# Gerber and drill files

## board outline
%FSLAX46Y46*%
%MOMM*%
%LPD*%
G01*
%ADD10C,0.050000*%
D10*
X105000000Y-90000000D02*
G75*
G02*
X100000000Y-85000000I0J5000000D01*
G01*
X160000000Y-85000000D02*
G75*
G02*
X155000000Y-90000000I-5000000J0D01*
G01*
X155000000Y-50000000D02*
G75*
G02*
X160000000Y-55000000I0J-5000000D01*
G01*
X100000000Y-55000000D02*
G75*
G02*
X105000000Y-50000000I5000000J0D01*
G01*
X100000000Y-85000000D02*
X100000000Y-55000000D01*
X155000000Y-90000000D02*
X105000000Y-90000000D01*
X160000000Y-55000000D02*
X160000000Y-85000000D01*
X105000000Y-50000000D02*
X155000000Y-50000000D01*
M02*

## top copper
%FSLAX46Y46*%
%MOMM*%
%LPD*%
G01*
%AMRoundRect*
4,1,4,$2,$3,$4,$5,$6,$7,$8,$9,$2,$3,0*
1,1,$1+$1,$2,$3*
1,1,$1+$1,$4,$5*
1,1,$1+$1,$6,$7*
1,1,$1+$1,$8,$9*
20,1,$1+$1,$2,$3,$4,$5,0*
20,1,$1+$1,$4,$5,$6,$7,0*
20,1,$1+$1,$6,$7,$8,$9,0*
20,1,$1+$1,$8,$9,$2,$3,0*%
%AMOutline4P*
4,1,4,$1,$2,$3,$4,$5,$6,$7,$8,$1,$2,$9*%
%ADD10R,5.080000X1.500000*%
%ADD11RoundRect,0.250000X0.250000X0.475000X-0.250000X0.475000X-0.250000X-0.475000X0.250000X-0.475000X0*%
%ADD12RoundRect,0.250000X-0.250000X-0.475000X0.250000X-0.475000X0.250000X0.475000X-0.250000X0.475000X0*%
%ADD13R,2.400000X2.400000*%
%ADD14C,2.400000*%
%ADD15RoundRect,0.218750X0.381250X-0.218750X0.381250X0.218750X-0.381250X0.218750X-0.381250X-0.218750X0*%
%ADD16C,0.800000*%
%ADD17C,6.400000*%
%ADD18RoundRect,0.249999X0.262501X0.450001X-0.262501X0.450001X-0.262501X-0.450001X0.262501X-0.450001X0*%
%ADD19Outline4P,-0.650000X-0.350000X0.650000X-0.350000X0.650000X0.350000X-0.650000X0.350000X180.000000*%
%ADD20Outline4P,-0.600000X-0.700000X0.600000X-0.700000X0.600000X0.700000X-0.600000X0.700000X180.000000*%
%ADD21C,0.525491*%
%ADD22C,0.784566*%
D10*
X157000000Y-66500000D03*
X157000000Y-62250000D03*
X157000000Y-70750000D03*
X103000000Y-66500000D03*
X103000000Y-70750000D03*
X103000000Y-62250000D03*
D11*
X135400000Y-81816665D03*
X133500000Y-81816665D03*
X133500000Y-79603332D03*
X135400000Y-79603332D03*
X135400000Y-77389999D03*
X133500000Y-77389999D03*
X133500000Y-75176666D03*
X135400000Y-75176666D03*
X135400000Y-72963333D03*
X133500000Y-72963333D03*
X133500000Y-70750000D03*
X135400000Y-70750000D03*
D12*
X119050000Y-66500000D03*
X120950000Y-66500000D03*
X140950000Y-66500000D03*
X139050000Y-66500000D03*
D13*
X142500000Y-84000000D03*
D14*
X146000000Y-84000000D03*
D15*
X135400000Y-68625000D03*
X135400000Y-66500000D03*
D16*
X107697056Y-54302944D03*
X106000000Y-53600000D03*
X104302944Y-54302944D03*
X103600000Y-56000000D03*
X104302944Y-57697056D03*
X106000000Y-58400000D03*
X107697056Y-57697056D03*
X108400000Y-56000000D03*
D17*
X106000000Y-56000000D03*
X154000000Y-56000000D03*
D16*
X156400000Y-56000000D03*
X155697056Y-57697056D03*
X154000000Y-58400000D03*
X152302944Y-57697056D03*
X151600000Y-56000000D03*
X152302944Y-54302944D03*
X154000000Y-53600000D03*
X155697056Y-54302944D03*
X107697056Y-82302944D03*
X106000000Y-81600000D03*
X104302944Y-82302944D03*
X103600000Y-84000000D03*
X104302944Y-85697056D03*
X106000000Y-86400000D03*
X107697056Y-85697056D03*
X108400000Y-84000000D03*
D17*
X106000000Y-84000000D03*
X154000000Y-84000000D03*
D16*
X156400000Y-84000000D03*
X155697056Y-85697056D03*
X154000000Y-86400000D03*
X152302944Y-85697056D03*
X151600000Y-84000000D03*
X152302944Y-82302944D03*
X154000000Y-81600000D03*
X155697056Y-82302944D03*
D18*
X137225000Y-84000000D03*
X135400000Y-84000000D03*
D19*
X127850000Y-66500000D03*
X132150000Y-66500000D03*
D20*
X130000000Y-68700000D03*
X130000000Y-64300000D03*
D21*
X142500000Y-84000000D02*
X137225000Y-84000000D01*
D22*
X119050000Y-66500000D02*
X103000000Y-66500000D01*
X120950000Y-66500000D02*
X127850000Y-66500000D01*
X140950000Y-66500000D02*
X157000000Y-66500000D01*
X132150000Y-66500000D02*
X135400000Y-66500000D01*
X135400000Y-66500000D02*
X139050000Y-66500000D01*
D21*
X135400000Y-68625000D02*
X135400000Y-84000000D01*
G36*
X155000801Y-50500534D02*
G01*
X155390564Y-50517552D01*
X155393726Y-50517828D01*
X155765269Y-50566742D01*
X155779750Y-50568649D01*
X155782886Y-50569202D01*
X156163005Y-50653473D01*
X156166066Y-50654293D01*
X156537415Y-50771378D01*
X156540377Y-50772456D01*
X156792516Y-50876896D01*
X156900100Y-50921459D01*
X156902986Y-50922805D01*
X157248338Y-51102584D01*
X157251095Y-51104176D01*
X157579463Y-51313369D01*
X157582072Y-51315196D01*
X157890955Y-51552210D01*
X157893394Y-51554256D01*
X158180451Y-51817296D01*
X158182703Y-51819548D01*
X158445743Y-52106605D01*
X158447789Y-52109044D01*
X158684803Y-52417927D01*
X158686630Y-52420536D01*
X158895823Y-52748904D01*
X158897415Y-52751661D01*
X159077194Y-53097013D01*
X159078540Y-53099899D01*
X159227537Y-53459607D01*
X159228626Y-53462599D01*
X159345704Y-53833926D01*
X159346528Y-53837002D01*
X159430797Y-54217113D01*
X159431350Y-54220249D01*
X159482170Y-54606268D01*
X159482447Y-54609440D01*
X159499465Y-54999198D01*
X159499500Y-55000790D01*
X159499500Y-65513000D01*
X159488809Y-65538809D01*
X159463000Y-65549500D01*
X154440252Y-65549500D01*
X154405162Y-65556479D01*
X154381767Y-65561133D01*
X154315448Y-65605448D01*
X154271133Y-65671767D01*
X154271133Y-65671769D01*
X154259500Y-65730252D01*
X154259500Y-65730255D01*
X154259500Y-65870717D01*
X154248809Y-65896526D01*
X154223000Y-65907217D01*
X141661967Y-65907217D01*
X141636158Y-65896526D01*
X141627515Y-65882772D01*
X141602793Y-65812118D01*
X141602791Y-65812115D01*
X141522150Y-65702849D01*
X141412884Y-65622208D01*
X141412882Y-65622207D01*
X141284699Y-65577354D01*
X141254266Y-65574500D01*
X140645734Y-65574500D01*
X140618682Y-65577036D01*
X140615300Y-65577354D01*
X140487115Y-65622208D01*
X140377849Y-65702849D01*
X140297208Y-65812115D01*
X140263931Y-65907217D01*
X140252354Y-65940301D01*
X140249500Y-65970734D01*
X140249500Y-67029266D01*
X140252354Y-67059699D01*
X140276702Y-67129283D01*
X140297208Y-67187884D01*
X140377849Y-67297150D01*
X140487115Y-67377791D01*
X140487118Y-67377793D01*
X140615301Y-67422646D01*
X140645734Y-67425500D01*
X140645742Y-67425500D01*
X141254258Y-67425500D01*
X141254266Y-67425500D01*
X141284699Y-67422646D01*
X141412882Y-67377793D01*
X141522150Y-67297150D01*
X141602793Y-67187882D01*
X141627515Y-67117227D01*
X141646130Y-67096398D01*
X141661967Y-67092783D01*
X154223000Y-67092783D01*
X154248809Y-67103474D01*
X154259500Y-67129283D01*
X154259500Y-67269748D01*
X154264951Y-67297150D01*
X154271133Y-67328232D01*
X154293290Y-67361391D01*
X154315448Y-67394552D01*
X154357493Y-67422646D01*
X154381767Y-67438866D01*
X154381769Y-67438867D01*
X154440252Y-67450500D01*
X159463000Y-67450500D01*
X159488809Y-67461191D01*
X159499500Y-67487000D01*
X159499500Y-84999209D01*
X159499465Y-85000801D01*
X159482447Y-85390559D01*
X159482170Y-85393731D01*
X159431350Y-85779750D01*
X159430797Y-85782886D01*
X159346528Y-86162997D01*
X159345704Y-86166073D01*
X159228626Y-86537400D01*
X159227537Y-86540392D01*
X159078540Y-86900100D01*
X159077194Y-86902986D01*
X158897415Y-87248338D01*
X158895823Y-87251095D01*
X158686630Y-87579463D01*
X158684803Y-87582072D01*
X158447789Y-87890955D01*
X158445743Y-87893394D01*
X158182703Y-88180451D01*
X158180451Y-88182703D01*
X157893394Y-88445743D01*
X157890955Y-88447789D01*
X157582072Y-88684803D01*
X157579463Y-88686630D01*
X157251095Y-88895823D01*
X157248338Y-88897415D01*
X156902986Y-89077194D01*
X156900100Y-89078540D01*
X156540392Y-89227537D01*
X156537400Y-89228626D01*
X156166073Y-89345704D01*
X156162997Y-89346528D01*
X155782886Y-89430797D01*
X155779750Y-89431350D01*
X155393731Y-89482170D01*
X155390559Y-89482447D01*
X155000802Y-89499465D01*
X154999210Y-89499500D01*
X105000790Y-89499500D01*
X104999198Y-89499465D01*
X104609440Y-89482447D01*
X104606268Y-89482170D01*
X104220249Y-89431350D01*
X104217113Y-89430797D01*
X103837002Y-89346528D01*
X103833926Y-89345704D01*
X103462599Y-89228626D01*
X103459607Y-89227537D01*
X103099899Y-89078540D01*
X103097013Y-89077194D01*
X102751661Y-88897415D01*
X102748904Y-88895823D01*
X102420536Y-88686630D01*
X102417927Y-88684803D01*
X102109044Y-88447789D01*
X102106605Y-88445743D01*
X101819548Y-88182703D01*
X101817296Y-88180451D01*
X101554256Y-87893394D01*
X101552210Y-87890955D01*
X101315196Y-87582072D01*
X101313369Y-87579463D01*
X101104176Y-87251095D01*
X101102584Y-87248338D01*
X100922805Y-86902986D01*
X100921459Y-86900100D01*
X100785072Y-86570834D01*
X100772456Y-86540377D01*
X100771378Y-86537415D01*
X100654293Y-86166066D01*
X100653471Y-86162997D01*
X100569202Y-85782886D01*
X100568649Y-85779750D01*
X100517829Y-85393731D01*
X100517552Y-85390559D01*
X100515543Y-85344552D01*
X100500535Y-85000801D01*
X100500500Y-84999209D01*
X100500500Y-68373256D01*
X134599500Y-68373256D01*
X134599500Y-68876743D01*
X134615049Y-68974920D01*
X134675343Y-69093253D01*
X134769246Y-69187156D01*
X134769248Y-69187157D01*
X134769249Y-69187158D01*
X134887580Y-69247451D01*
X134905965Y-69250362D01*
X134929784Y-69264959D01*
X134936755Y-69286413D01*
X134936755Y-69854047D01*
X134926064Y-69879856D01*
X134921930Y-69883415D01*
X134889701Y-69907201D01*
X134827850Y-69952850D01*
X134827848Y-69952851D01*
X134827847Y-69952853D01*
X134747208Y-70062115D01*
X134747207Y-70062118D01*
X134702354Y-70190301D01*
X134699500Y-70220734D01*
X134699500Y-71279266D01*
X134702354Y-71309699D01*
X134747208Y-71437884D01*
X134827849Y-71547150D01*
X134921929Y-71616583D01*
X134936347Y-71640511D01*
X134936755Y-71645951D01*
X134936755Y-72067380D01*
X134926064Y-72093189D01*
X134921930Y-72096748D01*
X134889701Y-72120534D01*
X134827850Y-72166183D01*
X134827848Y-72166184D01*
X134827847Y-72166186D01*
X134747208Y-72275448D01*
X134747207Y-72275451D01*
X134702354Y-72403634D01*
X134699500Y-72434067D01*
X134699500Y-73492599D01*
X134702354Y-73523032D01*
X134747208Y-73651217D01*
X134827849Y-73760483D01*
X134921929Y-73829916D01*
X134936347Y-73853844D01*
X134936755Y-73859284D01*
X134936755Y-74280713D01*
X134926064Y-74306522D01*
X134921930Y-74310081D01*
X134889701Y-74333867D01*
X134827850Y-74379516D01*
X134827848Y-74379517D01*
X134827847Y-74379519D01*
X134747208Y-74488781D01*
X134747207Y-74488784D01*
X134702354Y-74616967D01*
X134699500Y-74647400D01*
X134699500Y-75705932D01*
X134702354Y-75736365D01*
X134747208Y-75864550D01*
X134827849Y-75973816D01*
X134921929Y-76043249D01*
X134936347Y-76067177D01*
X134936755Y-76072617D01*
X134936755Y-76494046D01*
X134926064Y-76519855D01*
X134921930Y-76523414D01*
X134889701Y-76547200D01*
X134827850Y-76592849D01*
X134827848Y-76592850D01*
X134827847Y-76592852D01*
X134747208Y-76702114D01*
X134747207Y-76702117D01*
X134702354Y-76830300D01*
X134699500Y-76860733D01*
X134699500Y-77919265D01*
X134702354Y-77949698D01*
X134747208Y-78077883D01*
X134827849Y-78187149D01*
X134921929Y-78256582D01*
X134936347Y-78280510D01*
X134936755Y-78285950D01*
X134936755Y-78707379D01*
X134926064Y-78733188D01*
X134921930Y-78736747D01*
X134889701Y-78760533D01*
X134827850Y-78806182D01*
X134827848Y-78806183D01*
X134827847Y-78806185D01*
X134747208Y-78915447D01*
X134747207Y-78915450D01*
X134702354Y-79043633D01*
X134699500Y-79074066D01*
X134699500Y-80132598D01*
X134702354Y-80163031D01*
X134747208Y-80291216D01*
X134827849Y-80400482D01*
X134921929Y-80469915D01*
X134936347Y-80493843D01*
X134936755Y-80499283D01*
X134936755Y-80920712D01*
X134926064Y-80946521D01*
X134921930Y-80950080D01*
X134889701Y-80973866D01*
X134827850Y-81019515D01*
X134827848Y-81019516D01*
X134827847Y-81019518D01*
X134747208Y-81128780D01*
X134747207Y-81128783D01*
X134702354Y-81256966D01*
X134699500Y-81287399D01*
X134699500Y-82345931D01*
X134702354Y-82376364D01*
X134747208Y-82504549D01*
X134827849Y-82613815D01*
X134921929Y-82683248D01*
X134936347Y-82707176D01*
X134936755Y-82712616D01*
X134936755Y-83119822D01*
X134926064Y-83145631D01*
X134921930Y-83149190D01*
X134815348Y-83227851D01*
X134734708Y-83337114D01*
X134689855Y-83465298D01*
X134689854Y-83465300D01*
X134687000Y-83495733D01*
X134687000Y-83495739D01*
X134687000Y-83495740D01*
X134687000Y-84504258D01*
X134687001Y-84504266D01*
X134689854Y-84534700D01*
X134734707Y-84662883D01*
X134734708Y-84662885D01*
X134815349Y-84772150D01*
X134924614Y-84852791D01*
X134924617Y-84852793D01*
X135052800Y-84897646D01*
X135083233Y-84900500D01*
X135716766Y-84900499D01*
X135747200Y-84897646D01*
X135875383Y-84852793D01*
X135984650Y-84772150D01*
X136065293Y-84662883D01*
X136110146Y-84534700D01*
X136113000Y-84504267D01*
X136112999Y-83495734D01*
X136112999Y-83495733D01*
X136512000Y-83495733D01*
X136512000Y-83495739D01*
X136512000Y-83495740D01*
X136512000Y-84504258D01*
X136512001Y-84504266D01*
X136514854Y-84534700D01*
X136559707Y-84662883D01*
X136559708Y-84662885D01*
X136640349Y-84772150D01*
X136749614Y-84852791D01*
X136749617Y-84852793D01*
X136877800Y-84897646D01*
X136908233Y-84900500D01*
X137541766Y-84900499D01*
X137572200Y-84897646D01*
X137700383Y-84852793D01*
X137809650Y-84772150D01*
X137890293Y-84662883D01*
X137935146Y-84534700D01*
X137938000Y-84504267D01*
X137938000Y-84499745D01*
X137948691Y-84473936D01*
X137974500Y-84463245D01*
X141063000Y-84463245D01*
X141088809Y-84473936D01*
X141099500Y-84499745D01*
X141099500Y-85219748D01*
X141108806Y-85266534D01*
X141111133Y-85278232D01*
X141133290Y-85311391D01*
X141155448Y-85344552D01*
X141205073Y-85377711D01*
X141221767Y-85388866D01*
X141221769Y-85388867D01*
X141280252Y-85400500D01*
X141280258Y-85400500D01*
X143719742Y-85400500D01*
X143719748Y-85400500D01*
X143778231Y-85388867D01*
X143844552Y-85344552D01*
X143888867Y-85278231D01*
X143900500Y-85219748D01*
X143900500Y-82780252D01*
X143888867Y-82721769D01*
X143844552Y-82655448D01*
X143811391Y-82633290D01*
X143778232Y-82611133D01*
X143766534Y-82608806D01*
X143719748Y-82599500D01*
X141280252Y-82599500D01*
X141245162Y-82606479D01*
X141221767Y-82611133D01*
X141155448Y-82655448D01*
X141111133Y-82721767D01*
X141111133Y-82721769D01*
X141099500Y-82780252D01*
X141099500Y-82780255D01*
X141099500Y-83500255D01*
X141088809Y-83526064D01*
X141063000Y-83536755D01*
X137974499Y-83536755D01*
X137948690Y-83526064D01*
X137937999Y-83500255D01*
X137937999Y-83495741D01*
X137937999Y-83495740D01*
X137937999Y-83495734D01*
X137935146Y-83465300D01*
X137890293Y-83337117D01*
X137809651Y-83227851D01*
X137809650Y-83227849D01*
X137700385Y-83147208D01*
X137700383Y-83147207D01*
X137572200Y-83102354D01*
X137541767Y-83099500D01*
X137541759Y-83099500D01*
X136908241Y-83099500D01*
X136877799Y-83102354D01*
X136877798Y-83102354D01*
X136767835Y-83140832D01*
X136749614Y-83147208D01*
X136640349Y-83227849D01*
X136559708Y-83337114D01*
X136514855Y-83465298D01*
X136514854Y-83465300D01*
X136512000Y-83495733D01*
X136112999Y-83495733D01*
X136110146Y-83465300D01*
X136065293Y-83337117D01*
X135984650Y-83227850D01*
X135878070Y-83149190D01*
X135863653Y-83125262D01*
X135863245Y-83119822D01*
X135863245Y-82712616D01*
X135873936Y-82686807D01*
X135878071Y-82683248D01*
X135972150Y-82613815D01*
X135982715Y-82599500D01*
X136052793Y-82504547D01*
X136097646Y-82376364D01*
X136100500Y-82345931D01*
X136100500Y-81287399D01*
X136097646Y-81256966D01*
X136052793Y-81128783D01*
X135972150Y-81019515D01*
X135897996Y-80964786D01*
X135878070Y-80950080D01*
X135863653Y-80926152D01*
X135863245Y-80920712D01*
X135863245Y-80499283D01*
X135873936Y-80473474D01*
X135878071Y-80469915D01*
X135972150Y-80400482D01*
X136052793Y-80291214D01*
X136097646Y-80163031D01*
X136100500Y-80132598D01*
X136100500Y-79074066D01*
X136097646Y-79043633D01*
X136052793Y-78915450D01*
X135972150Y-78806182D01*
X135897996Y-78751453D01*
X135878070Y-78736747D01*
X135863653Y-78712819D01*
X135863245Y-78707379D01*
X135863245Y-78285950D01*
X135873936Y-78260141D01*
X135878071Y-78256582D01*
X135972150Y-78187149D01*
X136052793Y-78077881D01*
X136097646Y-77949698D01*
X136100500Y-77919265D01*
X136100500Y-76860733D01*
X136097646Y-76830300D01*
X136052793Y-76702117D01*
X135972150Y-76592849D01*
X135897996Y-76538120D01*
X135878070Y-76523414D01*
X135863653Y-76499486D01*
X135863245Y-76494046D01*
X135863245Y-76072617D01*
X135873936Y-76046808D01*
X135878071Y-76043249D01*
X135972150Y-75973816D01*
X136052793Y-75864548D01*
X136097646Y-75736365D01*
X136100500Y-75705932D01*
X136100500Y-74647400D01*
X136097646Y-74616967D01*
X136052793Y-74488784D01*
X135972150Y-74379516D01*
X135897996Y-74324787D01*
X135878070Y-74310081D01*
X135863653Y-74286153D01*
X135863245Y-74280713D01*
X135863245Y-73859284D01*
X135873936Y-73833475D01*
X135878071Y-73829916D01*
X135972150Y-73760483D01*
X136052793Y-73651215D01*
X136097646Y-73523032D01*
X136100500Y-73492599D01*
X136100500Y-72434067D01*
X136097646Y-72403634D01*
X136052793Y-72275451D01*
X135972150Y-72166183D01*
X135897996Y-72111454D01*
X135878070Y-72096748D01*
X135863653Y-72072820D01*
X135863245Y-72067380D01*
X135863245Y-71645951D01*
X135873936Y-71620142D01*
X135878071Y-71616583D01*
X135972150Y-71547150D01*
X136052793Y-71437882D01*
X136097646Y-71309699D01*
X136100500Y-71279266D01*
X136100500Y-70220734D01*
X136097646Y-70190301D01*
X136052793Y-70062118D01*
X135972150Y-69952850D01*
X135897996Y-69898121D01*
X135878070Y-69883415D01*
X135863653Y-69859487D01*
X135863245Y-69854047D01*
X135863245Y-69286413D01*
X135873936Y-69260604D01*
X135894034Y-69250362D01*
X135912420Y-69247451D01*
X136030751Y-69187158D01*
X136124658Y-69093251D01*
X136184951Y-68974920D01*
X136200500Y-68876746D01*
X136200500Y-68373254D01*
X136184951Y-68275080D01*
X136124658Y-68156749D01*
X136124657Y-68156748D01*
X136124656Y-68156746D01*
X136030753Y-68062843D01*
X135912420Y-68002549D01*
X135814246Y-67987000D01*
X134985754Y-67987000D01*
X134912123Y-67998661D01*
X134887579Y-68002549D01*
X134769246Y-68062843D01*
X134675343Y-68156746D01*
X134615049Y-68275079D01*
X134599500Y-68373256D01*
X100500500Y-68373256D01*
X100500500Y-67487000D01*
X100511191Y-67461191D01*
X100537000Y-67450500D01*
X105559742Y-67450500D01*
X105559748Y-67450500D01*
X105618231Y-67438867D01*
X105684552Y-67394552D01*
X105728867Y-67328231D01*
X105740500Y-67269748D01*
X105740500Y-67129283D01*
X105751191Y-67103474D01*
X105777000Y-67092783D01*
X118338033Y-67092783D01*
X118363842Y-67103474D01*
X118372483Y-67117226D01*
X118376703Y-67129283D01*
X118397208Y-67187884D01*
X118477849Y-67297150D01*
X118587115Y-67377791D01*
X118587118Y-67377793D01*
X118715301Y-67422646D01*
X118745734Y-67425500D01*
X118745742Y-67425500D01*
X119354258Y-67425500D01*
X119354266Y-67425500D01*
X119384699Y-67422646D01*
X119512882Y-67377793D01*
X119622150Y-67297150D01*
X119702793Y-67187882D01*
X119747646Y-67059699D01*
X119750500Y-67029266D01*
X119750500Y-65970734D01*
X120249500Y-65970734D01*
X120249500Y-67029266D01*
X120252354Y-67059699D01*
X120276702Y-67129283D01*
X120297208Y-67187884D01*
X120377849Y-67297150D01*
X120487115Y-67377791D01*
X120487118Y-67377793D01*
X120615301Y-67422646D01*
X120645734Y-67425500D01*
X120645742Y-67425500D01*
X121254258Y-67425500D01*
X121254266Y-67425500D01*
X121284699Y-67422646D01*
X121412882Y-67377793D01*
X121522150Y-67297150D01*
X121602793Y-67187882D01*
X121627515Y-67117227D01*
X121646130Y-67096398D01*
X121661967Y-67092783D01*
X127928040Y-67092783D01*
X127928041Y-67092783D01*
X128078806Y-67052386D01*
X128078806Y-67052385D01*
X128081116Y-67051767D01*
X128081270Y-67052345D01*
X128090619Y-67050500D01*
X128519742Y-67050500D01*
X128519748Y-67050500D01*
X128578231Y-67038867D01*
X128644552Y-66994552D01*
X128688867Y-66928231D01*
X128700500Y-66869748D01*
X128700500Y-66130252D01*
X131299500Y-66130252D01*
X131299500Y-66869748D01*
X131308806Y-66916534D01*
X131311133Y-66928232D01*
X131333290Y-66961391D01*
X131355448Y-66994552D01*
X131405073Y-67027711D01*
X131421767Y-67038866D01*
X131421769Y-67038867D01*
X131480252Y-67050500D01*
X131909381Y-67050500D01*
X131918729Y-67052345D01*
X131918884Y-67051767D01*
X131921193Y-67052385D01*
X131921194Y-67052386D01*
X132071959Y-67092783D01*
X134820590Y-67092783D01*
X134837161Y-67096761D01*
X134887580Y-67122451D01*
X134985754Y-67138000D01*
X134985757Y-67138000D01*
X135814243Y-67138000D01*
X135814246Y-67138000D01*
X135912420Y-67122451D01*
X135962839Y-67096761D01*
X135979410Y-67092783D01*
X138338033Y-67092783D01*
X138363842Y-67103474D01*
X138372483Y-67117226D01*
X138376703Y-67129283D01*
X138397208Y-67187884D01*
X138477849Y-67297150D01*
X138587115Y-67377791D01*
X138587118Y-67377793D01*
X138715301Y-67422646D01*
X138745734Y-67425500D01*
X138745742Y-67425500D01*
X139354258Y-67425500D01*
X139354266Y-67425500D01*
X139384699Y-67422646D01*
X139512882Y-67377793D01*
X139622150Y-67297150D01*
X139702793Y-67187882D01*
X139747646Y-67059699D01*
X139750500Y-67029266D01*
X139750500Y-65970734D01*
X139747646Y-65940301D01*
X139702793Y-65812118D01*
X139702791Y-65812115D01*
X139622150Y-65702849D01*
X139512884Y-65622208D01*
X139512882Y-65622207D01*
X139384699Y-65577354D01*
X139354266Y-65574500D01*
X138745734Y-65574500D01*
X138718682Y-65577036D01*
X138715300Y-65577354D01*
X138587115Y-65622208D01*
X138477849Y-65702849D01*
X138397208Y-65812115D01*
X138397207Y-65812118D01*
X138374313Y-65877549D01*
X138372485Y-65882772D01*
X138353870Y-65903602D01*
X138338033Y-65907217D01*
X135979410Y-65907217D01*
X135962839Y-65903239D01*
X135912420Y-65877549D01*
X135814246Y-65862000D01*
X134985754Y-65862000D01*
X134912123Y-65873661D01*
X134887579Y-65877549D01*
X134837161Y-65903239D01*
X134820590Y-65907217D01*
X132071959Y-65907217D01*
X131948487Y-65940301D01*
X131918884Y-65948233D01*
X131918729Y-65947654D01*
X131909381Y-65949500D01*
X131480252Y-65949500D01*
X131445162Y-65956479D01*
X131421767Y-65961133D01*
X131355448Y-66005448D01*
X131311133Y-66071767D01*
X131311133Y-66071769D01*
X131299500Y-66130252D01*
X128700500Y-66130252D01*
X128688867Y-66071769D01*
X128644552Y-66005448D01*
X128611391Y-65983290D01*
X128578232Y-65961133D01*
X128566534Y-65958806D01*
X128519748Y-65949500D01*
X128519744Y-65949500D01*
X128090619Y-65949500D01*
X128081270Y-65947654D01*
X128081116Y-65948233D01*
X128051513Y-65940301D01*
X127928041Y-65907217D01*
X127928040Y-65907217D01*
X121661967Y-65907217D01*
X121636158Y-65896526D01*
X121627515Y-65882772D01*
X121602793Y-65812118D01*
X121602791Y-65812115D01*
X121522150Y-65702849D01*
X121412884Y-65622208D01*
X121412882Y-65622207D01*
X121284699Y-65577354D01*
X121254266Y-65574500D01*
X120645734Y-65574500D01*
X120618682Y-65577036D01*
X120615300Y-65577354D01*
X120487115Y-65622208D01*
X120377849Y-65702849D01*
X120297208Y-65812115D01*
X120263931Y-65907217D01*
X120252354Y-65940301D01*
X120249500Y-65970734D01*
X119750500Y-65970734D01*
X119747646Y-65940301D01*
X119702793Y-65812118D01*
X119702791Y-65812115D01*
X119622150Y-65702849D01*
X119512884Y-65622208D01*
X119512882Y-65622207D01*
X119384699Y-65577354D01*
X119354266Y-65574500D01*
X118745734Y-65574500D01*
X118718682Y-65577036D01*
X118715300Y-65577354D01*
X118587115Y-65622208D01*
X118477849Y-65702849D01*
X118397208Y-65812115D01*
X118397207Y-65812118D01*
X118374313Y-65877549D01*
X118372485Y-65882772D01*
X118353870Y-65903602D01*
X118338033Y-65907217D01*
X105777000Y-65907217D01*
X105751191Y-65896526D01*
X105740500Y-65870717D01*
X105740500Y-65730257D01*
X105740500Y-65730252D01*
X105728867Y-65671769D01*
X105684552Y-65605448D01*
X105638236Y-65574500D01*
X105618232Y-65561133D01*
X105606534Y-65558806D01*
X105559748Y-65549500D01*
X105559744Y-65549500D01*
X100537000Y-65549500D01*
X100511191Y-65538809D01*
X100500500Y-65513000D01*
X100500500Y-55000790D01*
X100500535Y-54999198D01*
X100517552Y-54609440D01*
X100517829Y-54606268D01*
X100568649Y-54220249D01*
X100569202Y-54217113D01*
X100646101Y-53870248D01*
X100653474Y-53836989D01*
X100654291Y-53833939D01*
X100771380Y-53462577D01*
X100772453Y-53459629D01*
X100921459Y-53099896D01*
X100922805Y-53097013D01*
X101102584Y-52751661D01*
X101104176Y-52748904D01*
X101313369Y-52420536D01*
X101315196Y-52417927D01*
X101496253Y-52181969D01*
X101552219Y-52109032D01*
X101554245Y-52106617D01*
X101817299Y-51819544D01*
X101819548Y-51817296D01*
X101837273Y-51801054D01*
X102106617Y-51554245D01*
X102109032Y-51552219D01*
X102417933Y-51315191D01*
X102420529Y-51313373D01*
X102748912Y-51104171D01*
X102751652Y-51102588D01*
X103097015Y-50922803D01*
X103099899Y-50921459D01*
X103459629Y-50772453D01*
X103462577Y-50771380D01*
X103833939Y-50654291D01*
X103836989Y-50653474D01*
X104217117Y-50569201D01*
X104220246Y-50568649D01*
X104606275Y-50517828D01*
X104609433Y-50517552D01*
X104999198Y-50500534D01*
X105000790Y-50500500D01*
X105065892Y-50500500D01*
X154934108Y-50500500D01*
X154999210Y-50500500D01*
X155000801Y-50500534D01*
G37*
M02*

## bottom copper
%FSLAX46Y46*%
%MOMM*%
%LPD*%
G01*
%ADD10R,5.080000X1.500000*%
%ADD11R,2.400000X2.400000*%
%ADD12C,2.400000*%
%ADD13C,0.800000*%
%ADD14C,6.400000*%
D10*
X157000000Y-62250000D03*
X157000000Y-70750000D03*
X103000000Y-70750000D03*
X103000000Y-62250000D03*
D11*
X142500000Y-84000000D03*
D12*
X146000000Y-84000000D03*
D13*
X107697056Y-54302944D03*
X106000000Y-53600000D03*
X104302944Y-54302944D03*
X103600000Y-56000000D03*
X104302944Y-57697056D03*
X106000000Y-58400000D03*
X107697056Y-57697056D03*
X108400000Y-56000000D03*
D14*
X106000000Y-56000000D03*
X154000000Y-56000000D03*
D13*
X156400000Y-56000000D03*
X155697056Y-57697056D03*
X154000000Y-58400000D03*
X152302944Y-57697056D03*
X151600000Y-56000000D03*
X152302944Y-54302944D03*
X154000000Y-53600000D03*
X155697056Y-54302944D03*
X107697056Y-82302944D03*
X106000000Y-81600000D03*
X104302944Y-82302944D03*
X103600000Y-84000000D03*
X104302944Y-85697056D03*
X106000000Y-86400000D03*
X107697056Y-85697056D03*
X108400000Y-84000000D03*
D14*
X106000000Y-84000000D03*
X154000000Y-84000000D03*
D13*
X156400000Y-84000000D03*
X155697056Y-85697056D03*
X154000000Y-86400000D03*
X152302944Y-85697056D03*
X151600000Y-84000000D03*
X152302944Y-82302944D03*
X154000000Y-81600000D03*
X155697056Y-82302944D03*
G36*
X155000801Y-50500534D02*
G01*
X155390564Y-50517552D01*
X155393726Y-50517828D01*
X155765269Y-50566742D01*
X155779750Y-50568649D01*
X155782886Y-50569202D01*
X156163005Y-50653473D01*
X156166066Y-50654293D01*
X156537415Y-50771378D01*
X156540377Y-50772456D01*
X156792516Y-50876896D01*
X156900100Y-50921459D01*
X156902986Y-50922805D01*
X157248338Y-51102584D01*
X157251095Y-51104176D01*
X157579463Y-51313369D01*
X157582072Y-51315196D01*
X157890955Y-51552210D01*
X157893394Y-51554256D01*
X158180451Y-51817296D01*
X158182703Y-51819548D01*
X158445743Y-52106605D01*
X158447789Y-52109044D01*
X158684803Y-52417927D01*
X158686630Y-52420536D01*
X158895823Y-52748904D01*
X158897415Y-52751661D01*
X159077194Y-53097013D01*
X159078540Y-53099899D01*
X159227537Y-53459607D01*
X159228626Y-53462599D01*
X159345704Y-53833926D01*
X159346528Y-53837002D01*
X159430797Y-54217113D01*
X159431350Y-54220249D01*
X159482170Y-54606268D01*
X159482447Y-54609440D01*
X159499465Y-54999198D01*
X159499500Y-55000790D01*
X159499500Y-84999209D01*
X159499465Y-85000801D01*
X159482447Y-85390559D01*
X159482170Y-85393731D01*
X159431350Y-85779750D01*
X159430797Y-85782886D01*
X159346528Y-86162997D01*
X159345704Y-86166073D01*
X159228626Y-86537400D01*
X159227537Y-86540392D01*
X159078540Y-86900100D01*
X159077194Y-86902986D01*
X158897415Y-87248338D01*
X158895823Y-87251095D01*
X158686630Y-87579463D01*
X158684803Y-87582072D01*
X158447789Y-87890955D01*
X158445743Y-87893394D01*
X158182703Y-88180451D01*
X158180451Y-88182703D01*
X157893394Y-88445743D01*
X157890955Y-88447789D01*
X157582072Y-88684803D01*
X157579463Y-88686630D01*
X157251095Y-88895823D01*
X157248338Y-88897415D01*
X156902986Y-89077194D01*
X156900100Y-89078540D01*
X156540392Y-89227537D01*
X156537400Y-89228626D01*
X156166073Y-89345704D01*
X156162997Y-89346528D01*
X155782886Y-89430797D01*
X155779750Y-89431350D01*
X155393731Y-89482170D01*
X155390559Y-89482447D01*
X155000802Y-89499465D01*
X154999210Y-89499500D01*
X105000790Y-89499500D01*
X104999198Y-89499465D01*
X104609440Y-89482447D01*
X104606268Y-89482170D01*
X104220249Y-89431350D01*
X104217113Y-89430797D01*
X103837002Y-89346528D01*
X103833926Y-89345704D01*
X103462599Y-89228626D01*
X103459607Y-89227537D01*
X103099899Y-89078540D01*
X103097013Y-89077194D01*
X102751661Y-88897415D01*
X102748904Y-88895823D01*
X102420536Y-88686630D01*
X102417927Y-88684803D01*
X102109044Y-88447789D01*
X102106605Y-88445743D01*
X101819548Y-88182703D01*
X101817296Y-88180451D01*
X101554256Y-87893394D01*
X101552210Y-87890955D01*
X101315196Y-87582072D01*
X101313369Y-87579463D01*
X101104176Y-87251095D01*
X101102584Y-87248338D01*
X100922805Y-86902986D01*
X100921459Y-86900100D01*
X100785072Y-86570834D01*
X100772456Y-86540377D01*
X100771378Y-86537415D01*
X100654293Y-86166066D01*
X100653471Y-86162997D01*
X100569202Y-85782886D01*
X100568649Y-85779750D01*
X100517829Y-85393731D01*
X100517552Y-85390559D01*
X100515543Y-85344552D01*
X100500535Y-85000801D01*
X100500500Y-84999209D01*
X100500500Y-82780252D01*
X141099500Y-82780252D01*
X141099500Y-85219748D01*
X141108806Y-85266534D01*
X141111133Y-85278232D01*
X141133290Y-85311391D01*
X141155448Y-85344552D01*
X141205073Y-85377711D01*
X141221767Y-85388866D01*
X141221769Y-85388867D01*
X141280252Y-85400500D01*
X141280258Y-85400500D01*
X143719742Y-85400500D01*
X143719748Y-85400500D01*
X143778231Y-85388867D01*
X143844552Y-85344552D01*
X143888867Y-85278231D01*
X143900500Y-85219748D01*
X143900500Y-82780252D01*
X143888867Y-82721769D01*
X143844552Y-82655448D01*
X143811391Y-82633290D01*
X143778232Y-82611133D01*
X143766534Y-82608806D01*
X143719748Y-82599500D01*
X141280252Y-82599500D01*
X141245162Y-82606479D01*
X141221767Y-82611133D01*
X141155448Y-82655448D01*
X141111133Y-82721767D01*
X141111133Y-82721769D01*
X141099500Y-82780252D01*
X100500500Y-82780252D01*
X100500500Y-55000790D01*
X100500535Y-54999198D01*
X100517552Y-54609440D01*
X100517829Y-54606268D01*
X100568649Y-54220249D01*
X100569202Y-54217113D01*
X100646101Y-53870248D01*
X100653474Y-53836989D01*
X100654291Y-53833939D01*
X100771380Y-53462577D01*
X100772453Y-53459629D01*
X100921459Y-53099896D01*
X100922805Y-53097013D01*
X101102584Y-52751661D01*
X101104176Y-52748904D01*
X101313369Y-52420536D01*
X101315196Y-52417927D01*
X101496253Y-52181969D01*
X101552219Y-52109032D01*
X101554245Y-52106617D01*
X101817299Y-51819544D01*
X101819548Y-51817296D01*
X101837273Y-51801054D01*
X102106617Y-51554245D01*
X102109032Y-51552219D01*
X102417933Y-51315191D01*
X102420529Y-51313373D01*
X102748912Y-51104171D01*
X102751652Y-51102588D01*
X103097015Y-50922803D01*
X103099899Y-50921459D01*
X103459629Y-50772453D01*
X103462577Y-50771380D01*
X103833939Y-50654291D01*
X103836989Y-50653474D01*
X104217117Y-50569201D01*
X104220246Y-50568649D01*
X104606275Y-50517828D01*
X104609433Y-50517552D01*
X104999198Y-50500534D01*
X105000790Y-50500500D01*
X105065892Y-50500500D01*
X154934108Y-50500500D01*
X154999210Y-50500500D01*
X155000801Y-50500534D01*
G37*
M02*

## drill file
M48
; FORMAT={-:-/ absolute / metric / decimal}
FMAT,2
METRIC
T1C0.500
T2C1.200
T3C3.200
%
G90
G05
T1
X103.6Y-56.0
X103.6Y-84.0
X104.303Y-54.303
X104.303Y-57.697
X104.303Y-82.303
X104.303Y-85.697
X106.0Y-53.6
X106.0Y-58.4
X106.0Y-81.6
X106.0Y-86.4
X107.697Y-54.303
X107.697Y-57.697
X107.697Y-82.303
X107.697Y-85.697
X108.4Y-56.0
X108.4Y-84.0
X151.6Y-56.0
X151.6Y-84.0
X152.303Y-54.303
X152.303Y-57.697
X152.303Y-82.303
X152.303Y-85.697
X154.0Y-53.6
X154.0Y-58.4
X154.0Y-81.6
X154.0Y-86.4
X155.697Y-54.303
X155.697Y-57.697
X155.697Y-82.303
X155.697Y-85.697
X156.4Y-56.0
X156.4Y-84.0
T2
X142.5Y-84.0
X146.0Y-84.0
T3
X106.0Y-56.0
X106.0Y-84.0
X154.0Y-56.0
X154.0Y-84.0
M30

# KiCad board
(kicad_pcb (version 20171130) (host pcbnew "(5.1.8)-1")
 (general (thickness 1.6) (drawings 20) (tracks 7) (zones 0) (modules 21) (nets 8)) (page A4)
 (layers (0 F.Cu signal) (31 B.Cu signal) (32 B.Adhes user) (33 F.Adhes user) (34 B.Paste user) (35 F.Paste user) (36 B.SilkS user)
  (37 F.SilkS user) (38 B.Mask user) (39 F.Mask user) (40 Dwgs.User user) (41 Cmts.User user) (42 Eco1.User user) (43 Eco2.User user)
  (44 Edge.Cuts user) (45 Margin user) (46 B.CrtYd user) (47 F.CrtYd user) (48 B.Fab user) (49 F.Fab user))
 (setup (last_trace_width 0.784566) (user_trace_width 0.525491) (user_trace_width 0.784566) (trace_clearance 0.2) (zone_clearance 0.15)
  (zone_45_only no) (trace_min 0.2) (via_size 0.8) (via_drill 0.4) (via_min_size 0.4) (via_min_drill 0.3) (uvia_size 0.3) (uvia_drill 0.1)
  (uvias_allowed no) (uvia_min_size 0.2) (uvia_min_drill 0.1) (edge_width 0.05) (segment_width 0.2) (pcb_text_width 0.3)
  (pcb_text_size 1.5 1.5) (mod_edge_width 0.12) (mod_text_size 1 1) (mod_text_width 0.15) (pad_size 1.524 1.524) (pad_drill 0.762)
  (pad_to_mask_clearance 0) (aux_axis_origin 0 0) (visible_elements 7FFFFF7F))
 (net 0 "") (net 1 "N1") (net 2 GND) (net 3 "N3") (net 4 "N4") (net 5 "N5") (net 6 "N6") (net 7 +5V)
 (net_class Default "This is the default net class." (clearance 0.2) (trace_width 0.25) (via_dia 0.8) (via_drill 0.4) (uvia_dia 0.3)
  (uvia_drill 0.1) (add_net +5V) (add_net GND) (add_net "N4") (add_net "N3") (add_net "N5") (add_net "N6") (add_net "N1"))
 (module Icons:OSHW (layer F.Cu) (at 116 75)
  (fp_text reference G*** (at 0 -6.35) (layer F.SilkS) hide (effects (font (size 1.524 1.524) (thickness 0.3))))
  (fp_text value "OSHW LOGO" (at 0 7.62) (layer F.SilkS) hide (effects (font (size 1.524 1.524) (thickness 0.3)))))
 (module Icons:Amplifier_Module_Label (layer F.Cu) (at 130 55.99889)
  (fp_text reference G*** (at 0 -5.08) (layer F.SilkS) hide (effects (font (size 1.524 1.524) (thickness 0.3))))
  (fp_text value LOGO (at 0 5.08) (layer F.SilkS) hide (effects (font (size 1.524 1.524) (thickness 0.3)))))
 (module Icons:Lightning (layer F.Cu) (at 144.25 78.5)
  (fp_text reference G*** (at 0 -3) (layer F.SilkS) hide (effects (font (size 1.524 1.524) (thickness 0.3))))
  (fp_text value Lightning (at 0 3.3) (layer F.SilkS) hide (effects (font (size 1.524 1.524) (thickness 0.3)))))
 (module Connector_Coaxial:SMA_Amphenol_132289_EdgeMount (layer F.Cu) (at 157 66.5)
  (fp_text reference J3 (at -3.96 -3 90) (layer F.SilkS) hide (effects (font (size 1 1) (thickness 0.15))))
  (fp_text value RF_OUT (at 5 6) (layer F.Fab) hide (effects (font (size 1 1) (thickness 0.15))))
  (pad 1 smd rect (at 0 0 90) (size 1.5 5.08) (layers F.Cu F.Paste F.Mask) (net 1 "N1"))
  (pad 2 smd rect (at 0 -4.25 90) (size 1.5 5.08) (layers F.Cu F.Paste F.Mask) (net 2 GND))
  (pad 2 smd rect (at 0 4.25 90) (size 1.5 5.08) (layers F.Cu F.Paste F.Mask) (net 2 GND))
  (pad 2 smd rect (at 0 -4.25 90) (size 1.5 5.08) (layers B.Cu B.Paste B.Mask) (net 2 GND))
  (pad 2 smd rect (at 0 4.25 90) (size 1.5 5.08) (layers B.Cu B.Paste B.Mask) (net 2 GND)))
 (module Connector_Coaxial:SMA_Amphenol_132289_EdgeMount (layer F.Cu) (at 103 66.5 180)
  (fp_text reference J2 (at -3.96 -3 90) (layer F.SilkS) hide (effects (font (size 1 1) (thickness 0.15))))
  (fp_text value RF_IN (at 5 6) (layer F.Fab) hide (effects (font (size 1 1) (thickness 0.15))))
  (pad 1 smd rect (at 0 0 270) (size 1.5 5.08) (layers F.Cu F.Paste F.Mask) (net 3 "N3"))
  (pad 2 smd rect (at 0 -4.25 270) (size 1.5 5.08) (layers F.Cu F.Paste F.Mask) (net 2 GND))
  (pad 2 smd rect (at 0 4.25 270) (size 1.5 5.08) (layers F.Cu F.Paste F.Mask) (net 2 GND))
  (pad 2 smd rect (at 0 -4.25 270) (size 1.5 5.08) (layers B.Cu B.Paste B.Mask) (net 2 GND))
  (pad 2 smd rect (at 0 4.25 270) (size 1.5 5.08) (layers B.Cu B.Paste B.Mask) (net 2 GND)))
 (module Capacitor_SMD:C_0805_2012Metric (layer F.Cu) (at 134.45 81.816665 180)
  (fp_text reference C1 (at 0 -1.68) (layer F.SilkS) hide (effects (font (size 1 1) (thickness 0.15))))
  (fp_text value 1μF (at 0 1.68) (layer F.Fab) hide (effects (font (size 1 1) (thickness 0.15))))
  (pad 1 smd roundrect (at -0.95 0 180) (size 1 1.45) (layers F.Cu F.Paste F.Mask) (roundrect_rratio 0.25) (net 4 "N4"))
  (pad 2 smd roundrect (at 0.95 0 180) (size 1 1.45) (layers F.Cu F.Paste F.Mask) (roundrect_rratio 0.25) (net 2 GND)))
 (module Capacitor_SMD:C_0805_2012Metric (layer F.Cu) (at 134.45 79.603332 180)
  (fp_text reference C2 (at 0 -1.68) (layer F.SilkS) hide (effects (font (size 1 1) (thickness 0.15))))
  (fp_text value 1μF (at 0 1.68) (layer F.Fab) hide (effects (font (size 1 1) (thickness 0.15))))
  (pad 2 smd roundrect (at 0.95 0 180) (size 1 1.45) (layers F.Cu F.Paste F.Mask) (roundrect_rratio 0.25) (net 2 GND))
  (pad 1 smd roundrect (at -0.95 0 180) (size 1 1.45) (layers F.Cu F.Paste F.Mask) (roundrect_rratio 0.25) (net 4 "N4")))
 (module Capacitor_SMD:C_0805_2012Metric (layer F.Cu) (at 134.45 77.389999 180)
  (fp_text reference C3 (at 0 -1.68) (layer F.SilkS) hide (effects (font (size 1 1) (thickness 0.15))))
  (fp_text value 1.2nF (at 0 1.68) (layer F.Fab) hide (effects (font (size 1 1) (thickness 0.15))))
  (pad 1 smd roundrect (at -0.95 0 180) (size 1 1.45) (layers F.Cu F.Paste F.Mask) (roundrect_rratio 0.25) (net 4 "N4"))
  (pad 2 smd roundrect (at 0.95 0 180) (size 1 1.45) (layers F.Cu F.Paste F.Mask) (roundrect_rratio 0.25) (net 2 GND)))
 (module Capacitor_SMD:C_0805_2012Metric (layer F.Cu) (at 134.45 75.176666 180)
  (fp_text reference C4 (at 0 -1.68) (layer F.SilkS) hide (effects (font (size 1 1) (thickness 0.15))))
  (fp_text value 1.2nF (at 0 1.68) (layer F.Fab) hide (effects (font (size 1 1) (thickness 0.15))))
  (pad 2 smd roundrect (at 0.95 0 180) (size 1 1.45) (layers F.Cu F.Paste F.Mask) (roundrect_rratio 0.25) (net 2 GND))
  (pad 1 smd roundrect (at -0.95 0 180) (size 1 1.45) (layers F.Cu F.Paste F.Mask) (roundrect_rratio 0.25) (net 4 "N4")))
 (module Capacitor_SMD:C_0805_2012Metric (layer F.Cu) (at 134.45 72.963333 180)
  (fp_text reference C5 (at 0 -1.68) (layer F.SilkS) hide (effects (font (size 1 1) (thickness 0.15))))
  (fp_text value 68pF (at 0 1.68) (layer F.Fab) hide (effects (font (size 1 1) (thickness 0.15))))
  (pad 1 smd roundrect (at -0.95 0 180) (size 1 1.45) (layers F.Cu F.Paste F.Mask) (roundrect_rratio 0.25) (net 4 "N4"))
  (pad 2 smd roundrect (at 0.95 0 180) (size 1 1.45) (layers F.Cu F.Paste F.Mask) (roundrect_rratio 0.25) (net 2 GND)))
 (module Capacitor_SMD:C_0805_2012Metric (layer F.Cu) (at 134.45 70.75 180)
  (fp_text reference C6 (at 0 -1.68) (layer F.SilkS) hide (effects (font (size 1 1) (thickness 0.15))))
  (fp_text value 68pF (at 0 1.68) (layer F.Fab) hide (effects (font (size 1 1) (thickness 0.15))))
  (pad 2 smd roundrect (at 0.95 0 180) (size 1 1.45) (layers F.Cu F.Paste F.Mask) (roundrect_rratio 0.25) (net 2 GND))
  (pad 1 smd roundrect (at -0.95 0 180) (size 1 1.45) (layers F.Cu F.Paste F.Mask) (roundrect_rratio 0.25) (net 4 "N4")))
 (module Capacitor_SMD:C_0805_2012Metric (layer F.Cu) (at 120 66.5)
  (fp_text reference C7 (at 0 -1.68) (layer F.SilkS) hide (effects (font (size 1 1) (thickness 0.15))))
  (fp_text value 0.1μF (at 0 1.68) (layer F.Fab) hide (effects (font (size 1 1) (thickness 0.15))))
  (pad 1 smd roundrect (at -0.95 0) (size 1 1.45) (layers F.Cu F.Paste F.Mask) (roundrect_rratio 0.25) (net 3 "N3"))
  (pad 2 smd roundrect (at 0.95 0) (size 1 1.45) (layers F.Cu F.Paste F.Mask) (roundrect_rratio 0.25) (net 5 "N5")))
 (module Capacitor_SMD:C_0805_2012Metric (layer F.Cu) (at 140 66.5)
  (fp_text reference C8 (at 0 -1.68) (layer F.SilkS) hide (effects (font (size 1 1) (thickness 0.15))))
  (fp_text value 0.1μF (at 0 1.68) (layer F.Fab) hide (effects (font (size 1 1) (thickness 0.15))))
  (pad 2 smd roundrect (at 0.95 0) (size 1 1.45) (layers F.Cu F.Paste F.Mask) (roundrect_rratio 0.25) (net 1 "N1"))
  (pad 1 smd roundrect (at -0.95 0) (size 1 1.45) (layers F.Cu F.Paste F.Mask) (roundrect_rratio 0.25) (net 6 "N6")))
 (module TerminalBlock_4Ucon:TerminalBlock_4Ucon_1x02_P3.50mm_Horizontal (layer F.Cu) (at 142.5 84)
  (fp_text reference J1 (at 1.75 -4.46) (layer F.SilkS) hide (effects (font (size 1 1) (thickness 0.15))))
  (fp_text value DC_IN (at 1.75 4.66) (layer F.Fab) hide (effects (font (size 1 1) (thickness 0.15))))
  (pad 1 thru_hole rect (at 0 0) (size 2.4 2.4) (drill 1.2) (layers *.Cu *.Mask) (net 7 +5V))
  (pad 2 thru_hole circle (at 3.5 0) (size 2.4 2.4) (drill 1.2) (layers *.Cu *.Mask) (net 2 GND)))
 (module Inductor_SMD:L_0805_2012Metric (layer F.Cu) (at 135.4 67.5625 90)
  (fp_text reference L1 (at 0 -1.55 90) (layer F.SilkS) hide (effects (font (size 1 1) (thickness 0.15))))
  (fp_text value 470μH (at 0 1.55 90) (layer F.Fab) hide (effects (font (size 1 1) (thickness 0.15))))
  (pad 1 smd roundrect (at -1.0625 0 90) (size 0.875 1.2) (layers F.Cu F.Paste F.Mask) (roundrect_rratio 0.25) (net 4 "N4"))
  (pad 2 smd roundrect (at 1.0625 0 90) (size 0.875 1.2) (layers F.Cu F.Paste F.Mask) (roundrect_rratio 0.25) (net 6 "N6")))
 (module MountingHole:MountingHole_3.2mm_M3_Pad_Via (layer F.Cu) (at 106 56)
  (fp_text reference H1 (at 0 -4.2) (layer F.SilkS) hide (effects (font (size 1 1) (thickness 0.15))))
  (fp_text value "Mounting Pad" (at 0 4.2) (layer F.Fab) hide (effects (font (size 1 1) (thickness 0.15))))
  (pad 1 thru_hole circle (at 1.697056 -1.697056) (size 0.8 0.8) (drill 0.5) (layers *.Cu *.Mask) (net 2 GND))
  (pad 1 thru_hole circle (at 0 -2.4) (size 0.8 0.8) (drill 0.5) (layers *.Cu *.Mask) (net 2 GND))
  (pad 1 thru_hole circle (at -1.697056 -1.697056) (size 0.8 0.8) (drill 0.5) (layers *.Cu *.Mask) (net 2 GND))
  (pad 1 thru_hole circle (at -2.4 0) (size 0.8 0.8) (drill 0.5) (layers *.Cu *.Mask) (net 2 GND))
  (pad 1 thru_hole circle (at -1.697056 1.697056) (size 0.8 0.8) (drill 0.5) (layers *.Cu *.Mask) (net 2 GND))
  (pad 1 thru_hole circle (at 0 2.4) (size 0.8 0.8) (drill 0.5) (layers *.Cu *.Mask) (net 2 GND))
  (pad 1 thru_hole circle (at 1.697056 1.697056) (size 0.8 0.8) (drill 0.5) (layers *.Cu *.Mask) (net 2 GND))
  (pad 1 thru_hole circle (at 2.4 0) (size 0.8 0.8) (drill 0.5) (layers *.Cu *.Mask) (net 2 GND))
  (pad 1 thru_hole circle (at 0 0) (size 6.4 6.4) (drill 3.2) (layers *.Cu *.Mask) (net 2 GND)))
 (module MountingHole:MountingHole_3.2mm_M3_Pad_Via (layer F.Cu) (at 154 56)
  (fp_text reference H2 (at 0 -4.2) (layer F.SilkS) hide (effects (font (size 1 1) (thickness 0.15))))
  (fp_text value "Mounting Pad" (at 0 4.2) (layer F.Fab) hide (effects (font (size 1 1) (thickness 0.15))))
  (pad 1 thru_hole circle (at 0 0) (size 6.4 6.4) (drill 3.2) (layers *.Cu *.Mask) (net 2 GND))
  (pad 1 thru_hole circle (at 2.4 0) (size 0.8 0.8) (drill 0.5) (layers *.Cu *.Mask) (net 2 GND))
  (pad 1 thru_hole circle (at 1.697056 1.697056) (size 0.8 0.8) (drill 0.5) (layers *.Cu *.Mask) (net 2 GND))
  (pad 1 thru_hole circle (at 0 2.4) (size 0.8 0.8) (drill 0.5) (layers *.Cu *.Mask) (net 2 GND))
  (pad 1 thru_hole circle (at -1.697056 1.697056) (size 0.8 0.8) (drill 0.5) (layers *.Cu *.Mask) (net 2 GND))
  (pad 1 thru_hole circle (at -2.4 0) (size 0.8 0.8) (drill 0.5) (layers *.Cu *.Mask) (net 2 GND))
  (pad 1 thru_hole circle (at -1.697056 -1.697056) (size 0.8 0.8) (drill 0.5) (layers *.Cu *.Mask) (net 2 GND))
  (pad 1 thru_hole circle (at 0 -2.4) (size 0.8 0.8) (drill 0.5) (layers *.Cu *.Mask) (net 2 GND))
  (pad 1 thru_hole circle (at 1.697056 -1.697056) (size 0.8 0.8) (drill 0.5) (layers *.Cu *.Mask) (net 2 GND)))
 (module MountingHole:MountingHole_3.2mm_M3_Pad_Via (layer F.Cu) (at 106 84)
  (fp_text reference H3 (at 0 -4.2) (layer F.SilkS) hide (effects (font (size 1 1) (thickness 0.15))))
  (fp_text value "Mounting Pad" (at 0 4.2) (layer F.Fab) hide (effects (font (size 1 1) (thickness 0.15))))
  (pad 1 thru_hole circle (at 1.697056 -1.697056) (size 0.8 0.8) (drill 0.5) (layers *.Cu *.Mask) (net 2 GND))
  (pad 1 thru_hole circle (at 0 -2.4) (size 0.8 0.8) (drill 0.5) (layers *.Cu *.Mask) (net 2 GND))
  (pad 1 thru_hole circle (at -1.697056 -1.697056) (size 0.8 0.8) (drill 0.5) (layers *.Cu *.Mask) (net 2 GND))
  (pad 1 thru_hole circle (at -2.4 0) (size 0.8 0.8) (drill 0.5) (layers *.Cu *.Mask) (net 2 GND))
  (pad 1 thru_hole circle (at -1.697056 1.697056) (size 0.8 0.8) (drill 0.5) (layers *.Cu *.Mask) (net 2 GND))
  (pad 1 thru_hole circle (at 0 2.4) (size 0.8 0.8) (drill 0.5) (layers *.Cu *.Mask) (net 2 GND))
  (pad 1 thru_hole circle (at 1.697056 1.697056) (size 0.8 0.8) (drill 0.5) (layers *.Cu *.Mask) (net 2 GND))
  (pad 1 thru_hole circle (at 2.4 0) (size 0.8 0.8) (drill 0.5) (layers *.Cu *.Mask) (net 2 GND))
  (pad 1 thru_hole circle (at 0 0) (size 6.4 6.4) (drill 3.2) (layers *.Cu *.Mask) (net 2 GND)))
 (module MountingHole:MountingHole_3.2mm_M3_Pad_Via (layer F.Cu) (at 154 84)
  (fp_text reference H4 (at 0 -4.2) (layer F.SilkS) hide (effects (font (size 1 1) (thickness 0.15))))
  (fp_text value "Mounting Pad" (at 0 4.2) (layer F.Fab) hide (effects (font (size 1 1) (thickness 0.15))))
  (pad 1 thru_hole circle (at 0 0) (size 6.4 6.4) (drill 3.2) (layers *.Cu *.Mask) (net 2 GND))
  (pad 1 thru_hole circle (at 2.4 0) (size 0.8 0.8) (drill 0.5) (layers *.Cu *.Mask) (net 2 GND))
  (pad 1 thru_hole circle (at 1.697056 1.697056) (size 0.8 0.8) (drill 0.5) (layers *.Cu *.Mask) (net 2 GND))
  (pad 1 thru_hole circle (at 0 2.4) (size 0.8 0.8) (drill 0.5) (layers *.Cu *.Mask) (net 2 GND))
  (pad 1 thru_hole circle (at -1.697056 1.697056) (size 0.8 0.8) (drill 0.5) (layers *.Cu *.Mask) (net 2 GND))
  (pad 1 thru_hole circle (at -2.4 0) (size 0.8 0.8) (drill 0.5) (layers *.Cu *.Mask) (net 2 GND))
  (pad 1 thru_hole circle (at -1.697056 -1.697056) (size 0.8 0.8) (drill 0.5) (layers *.Cu *.Mask) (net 2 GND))
  (pad 1 thru_hole circle (at 0 -2.4) (size 0.8 0.8) (drill 0.5) (layers *.Cu *.Mask) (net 2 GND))
  (pad 1 thru_hole circle (at 1.697056 -1.697056) (size 0.8 0.8) (drill 0.5) (layers *.Cu *.Mask) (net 2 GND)))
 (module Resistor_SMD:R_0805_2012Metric (layer F.Cu) (at 136.3125 84 180)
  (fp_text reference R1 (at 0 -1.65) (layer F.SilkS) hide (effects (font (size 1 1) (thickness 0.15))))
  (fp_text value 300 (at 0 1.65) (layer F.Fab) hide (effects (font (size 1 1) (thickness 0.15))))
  (pad 1 smd roundrect (at -0.9125 0 180) (size 1.025 1.4) (layers F.Cu F.Paste F.Mask) (roundrect_rratio 0.2439014634146341) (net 7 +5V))
  (pad 2 smd roundrect (at 0.9125 0 180) (size 1.025 1.4) (layers F.Cu F.Paste F.Mask) (roundrect_rratio 0.2439014634146341) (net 4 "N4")))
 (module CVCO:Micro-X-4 (layer F.Cu) (at 130 66.5)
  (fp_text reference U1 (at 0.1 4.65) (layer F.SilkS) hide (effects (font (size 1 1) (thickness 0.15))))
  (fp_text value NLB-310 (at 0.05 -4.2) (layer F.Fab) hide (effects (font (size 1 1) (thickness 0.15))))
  (pad 1 smd trapezoid (at -2.15 0 180) (size 1.3 0.7) (layers F.Cu F.Paste F.Mask) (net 5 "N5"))
  (pad 3 smd trapezoid (at 2.15 0 180) (size 1.3 0.7) (layers F.Cu F.Paste F.Mask) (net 6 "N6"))
  (pad 2 smd trapezoid (at 0 2.2 180) (size 1.2 1.4) (layers F.Cu F.Paste F.Mask) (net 2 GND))
  (pad 4 smd trapezoid (at 0 -2.2 180) (size 1.2 1.4) (layers F.Cu F.Paste F.Mask) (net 2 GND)))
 (gr_arc (start 105 85) (end 100 85) (angle -90) (layer Edge.Cuts) (width 0.05))
 (gr_arc (start 155 85) (end 155 90) (angle -90) (layer Edge.Cuts) (width 0.05))
 (gr_arc (start 155 55) (end 160 55) (angle -90) (layer Edge.Cuts) (width 0.05))
 (gr_arc (start 105 55) (end 105 50) (angle -90) (layer Edge.Cuts) (width 0.05))
 (gr_line (start 100 85) (end 100 55) (layer Edge.Cuts) (width 0.05))
 (gr_line (start 155 90) (end 105 90) (layer Edge.Cuts) (width 0.05))
 (gr_line (start 160 55) (end 160 85) (layer Edge.Cuts) (width 0.05))
 (gr_line (start 105 50) (end 155 50) (layer Edge.Cuts) (width 0.05))
 (segment (start 142.5 84) (end 137.225 84) (width 0.525491) (layer F.Cu) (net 7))
 (segment (start 119.05 66.5) (end 103 66.5) (width 0.784566) (layer F.Cu) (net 3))
 (segment (start 120.95 66.5) (end 127.85 66.5) (width 0.784566) (layer F.Cu) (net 5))
 (segment (start 140.95 66.5) (end 157 66.5) (width 0.784566) (layer F.Cu) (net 1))
 (segment (start 132.15 66.5) (end 135.4 66.5) (width 0.784566) (layer F.Cu) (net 6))
 (segment (start 135.4 66.5) (end 139.05 66.5) (width 0.784566) (layer F.Cu) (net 6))
 (segment (start 135.4 68.625) (end 135.4 84) (width 0.525491) (layer F.Cu) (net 4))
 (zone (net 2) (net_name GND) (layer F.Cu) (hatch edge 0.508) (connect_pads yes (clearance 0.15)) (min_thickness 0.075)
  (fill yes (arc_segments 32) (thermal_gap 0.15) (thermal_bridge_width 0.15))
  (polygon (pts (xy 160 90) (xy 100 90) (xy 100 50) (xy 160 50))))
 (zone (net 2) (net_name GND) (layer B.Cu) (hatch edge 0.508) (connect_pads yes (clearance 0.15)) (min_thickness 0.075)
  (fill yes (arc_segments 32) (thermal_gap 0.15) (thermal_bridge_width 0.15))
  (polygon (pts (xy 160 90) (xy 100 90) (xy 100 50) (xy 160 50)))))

